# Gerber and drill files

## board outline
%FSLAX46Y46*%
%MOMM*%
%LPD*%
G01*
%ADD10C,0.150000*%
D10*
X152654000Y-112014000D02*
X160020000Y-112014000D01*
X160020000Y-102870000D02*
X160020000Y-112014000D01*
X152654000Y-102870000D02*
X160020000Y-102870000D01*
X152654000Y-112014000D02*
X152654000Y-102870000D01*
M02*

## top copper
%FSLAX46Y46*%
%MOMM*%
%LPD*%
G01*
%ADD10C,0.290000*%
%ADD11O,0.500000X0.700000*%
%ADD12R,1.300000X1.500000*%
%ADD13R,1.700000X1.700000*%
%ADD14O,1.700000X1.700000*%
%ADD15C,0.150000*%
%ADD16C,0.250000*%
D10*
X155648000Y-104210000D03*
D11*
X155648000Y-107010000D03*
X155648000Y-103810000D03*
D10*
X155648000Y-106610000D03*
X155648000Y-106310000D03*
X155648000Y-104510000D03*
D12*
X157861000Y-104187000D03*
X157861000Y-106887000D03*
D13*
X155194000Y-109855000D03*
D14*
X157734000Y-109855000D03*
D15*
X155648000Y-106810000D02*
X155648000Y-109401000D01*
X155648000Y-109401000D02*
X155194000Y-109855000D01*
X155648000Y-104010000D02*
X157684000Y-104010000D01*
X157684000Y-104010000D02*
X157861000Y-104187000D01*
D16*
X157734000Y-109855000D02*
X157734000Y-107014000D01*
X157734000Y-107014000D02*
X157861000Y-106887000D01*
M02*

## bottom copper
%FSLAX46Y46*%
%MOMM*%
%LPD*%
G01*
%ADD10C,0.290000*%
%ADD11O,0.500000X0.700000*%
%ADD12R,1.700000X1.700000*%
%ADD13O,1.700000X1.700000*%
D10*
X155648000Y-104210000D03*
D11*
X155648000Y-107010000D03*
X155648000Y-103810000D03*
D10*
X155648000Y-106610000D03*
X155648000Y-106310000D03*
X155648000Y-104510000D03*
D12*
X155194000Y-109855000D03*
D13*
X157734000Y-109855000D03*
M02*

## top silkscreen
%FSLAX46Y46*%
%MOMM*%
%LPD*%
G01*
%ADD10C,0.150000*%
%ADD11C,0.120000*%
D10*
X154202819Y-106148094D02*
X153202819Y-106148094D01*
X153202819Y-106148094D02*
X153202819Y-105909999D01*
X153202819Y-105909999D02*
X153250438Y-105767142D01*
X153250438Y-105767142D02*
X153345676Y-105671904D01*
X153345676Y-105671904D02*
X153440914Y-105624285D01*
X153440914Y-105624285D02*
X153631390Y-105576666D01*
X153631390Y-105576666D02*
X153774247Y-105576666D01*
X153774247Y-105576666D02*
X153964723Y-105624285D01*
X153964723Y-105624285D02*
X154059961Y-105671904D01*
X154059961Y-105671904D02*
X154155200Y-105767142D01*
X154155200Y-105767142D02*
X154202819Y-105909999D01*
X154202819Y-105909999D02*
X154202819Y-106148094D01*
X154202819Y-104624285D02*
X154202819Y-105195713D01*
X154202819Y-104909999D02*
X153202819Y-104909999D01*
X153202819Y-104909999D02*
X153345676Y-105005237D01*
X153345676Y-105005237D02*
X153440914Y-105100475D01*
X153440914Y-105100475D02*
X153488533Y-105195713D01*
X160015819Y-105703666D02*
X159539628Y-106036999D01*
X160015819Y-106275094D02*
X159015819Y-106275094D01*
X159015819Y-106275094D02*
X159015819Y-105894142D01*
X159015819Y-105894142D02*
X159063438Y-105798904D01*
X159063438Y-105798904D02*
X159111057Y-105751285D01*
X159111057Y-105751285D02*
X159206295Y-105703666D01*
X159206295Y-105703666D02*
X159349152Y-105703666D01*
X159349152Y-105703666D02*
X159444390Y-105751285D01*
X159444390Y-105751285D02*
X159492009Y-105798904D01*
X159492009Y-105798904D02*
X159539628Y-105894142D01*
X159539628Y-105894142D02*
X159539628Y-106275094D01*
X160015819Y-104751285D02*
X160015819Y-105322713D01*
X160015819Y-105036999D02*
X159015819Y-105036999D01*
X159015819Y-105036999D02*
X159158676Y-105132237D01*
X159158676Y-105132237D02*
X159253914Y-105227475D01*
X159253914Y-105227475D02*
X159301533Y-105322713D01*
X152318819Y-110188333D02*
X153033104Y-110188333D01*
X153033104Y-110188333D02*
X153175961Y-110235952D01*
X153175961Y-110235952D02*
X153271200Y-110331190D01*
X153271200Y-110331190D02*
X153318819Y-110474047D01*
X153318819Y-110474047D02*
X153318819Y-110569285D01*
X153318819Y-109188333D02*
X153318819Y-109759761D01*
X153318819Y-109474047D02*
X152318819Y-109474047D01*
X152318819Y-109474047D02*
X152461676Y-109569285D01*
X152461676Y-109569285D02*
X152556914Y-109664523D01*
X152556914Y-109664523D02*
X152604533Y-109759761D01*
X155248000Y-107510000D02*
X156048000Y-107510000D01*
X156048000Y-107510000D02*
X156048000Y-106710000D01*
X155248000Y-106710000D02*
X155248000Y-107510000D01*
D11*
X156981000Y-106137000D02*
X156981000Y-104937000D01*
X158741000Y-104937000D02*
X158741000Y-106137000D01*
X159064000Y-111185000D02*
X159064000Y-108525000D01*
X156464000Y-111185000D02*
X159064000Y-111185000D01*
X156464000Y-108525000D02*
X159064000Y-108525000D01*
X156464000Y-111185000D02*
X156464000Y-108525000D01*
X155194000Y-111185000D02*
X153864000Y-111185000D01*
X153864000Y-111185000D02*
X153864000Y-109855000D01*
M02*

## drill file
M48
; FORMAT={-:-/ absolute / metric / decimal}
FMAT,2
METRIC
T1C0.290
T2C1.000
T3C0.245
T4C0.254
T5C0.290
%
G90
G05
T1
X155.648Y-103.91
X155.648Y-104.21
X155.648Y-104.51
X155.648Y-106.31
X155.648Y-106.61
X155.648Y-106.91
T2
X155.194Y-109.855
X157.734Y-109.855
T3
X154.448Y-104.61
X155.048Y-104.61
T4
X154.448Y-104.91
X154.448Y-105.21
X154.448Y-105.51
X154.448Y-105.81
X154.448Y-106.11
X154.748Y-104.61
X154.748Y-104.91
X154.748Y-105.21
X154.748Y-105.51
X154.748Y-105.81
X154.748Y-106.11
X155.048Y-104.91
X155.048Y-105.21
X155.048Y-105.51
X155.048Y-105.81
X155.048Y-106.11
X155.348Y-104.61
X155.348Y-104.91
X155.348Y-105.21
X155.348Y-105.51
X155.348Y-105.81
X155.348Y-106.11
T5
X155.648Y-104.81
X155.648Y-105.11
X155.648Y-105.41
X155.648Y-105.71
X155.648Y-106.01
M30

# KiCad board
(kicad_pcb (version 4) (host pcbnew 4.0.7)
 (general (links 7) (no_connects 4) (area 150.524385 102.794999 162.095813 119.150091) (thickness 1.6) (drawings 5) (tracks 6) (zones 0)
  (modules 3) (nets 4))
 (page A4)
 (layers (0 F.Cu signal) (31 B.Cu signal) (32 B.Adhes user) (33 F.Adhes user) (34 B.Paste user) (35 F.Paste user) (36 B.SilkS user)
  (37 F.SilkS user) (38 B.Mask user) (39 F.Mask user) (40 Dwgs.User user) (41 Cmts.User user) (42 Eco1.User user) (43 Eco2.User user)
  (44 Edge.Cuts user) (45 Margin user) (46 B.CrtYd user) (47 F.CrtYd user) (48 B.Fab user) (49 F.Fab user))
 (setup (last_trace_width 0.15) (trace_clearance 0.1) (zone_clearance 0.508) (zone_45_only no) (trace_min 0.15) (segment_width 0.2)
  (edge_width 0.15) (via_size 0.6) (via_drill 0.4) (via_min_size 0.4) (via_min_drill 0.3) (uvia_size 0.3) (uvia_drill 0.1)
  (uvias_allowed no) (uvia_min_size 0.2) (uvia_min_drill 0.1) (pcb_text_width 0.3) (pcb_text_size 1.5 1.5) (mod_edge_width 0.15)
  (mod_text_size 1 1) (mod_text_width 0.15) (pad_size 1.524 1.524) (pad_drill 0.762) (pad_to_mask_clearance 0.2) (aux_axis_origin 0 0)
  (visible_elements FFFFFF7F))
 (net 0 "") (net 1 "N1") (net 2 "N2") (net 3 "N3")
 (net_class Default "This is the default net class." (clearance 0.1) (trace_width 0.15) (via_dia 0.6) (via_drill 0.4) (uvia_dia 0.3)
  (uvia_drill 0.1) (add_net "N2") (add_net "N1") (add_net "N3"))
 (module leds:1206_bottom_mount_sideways (layer F.Cu) (at 155.448 105.41 90)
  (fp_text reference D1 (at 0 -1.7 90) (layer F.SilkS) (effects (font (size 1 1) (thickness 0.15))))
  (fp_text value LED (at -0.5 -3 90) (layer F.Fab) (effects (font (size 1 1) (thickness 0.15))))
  (fp_line (start -2.1 -0.2) (end -2.1 0.6) (layer F.SilkS) (width 0.15))
  (fp_line (start -2.1 0.6) (end -1.3 0.6) (layer F.SilkS) (width 0.15))
  (fp_line (start -1.3 -0.2) (end -2.1 -0.2) (layer F.SilkS) (width 0.15))
  (pad 2 thru_hole circle (at 1.2 0.2 270) (size 0.29 0.29) (drill 0.29) (layers *.Cu *.Mask) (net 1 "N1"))
  (pad "" np_thru_hole circle (at 0.8 -0.7 270) (size 0.254 0.254) (drill 0.254) (layers *.Cu *.Mask))
  (pad "" np_thru_hole circle (at 0.5 -0.7 270) (size 0.254 0.254) (drill 0.254) (layers *.Cu *.Mask))
  (pad "" np_thru_hole circle (at 0.2 -0.7 270) (size 0.254 0.254) (drill 0.254) (layers *.Cu *.Mask))
  (pad "" np_thru_hole circle (at -0.1 -0.7 270) (size 0.254 0.254) (drill 0.254) (layers *.Cu *.Mask))
  (pad "" np_thru_hole circle (at -0.4 -0.7 270) (size 0.254 0.254) (drill 0.254) (layers *.Cu *.Mask))
  (pad "" np_thru_hole circle (at -0.7 -0.7 270) (size 0.254 0.254) (drill 0.254) (layers *.Cu *.Mask))
  (pad "" np_thru_hole circle (at 0.8 -0.4 270) (size 0.245 0.245) (drill 0.245) (layers *.Cu *.Mask))
  (pad 1 thru_hole oval (at -1.5 0.2 270) (size 0.7 0.5) (drill 0.29 (offset 0.1 0)) (layers *.Cu *.Mask) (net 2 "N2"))
  (pad 2 thru_hole oval (at 1.5 0.2 90) (size 0.7 0.5) (drill oval 0.29 (offset 0.1 0)) (layers *.Cu *.Mask) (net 1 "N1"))
  (pad "" np_thru_hole circle (at 0.8 -1 270) (size 0.245 0.245) (drill 0.245) (layers *.Cu *.Mask))
  (pad "" np_thru_hole circle (at 0.8 -0.1 270) (size 0.254 0.254) (drill 0.254) (layers *.Cu *.Mask))
  (pad "" np_thru_hole circle (at 0.5 -1 270) (size 0.254 0.254) (drill 0.254) (layers *.Cu *.Mask))
  (pad "" np_thru_hole circle (at 0.5 -0.4 270) (size 0.254 0.254) (drill 0.254) (layers *.Cu *.Mask))
  (pad "" np_thru_hole circle (at 0.5 -0.1 270) (size 0.254 0.254) (drill 0.254) (layers *.Cu *.Mask))
  (pad "" np_thru_hole circle (at 0.2 -1 270) (size 0.254 0.254) (drill 0.254) (layers *.Cu *.Mask))
  (pad "" np_thru_hole circle (at 0.2 -0.4 270) (size 0.254 0.254) (drill 0.254) (layers *.Cu *.Mask))
  (pad "" np_thru_hole circle (at 0.2 -0.1 270) (size 0.254 0.254) (drill 0.254) (layers *.Cu *.Mask))
  (pad "" np_thru_hole circle (at -0.1 -1 270) (size 0.254 0.254) (drill 0.254) (layers *.Cu *.Mask))
  (pad "" np_thru_hole circle (at -0.1 -0.4 270) (size 0.254 0.254) (drill 0.254) (layers *.Cu *.Mask))
  (pad "" np_thru_hole circle (at -0.1 -0.1 270) (size 0.254 0.254) (drill 0.254) (layers *.Cu *.Mask))
  (pad "" np_thru_hole circle (at -0.4 -1 270) (size 0.254 0.254) (drill 0.254) (layers *.Cu *.Mask))
  (pad "" np_thru_hole circle (at -0.4 -0.4 270) (size 0.254 0.254) (drill 0.254) (layers *.Cu *.Mask))
  (pad "" np_thru_hole circle (at -0.4 -0.1 270) (size 0.254 0.254) (drill 0.254) (layers *.Cu *.Mask))
  (pad "" np_thru_hole circle (at -0.7 -1 270) (size 0.254 0.254) (drill 0.254) (layers *.Cu *.Mask))
  (pad "" np_thru_hole circle (at -0.7 -0.4 270) (size 0.254 0.254) (drill 0.254) (layers *.Cu *.Mask))
  (pad "" np_thru_hole circle (at -0.7 -0.1 270) (size 0.254 0.254) (drill 0.254) (layers *.Cu *.Mask))
  (pad 1 thru_hole circle (at -1.2 0.2 270) (size 0.29 0.29) (drill 0.29) (layers *.Cu *.Mask) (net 2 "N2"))
  (pad 1 thru_hole circle (at -0.9 0.2 270) (size 0.29 0.29) (drill 0.29) (layers *.Cu *.Mask) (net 2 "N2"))
  (pad "" np_thru_hole circle (at -0.6 0.2 270) (size 0.29 0.29) (drill 0.29) (layers *.Cu *.Mask))
  (pad "" np_thru_hole circle (at -0.3 0.2 270) (size 0.29 0.29) (drill 0.29) (layers *.Cu *.Mask))
  (pad "" np_thru_hole circle (at 0 0.2 270) (size 0.29 0.29) (drill 0.29) (layers *.Cu *.Mask))
  (pad "" np_thru_hole circle (at 0.3 0.2 270) (size 0.29 0.29) (drill 0.29) (layers *.Cu *.Mask))
  (pad "" np_thru_hole circle (at 0.6 0.2 270) (size 0.29 0.29) (drill 0.29) (layers *.Cu *.Mask))
  (pad 2 thru_hole circle (at 0.9 0.2 270) (size 0.29 0.29) (drill 0.29) (layers *.Cu *.Mask) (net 1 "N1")))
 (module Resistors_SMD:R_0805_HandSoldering (layer F.Cu) (at 157.861 105.537 270)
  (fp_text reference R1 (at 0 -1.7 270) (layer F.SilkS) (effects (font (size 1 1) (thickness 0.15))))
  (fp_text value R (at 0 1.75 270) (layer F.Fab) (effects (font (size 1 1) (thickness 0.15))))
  (fp_line (start 0.6 0.88) (end -0.6 0.88) (layer F.SilkS) (width 0.12))
  (fp_line (start -0.6 -0.88) (end 0.6 -0.88) (layer F.SilkS) (width 0.12))
  (pad 1 smd rect (at -1.35 0 270) (size 1.5 1.3) (layers F.Cu F.Paste F.Mask) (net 1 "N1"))
  (pad 2 smd rect (at 1.35 0 270) (size 1.5 1.3) (layers F.Cu F.Paste F.Mask) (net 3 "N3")))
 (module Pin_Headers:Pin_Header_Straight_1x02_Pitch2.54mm (layer F.Cu) (at 155.194 109.855 90)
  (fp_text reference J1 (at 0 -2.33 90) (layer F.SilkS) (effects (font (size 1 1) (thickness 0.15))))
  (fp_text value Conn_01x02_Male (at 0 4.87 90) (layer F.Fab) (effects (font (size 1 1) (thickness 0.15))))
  (fp_line (start -1.33 3.87) (end 1.33 3.87) (layer F.SilkS) (width 0.12))
  (fp_line (start -1.33 1.27) (end -1.33 3.87) (layer F.SilkS) (width 0.12))
  (fp_line (start 1.33 1.27) (end 1.33 3.87) (layer F.SilkS) (width 0.12))
  (fp_line (start -1.33 1.27) (end 1.33 1.27) (layer F.SilkS) (width 0.12))
  (fp_line (start -1.33 0) (end -1.33 -1.33) (layer F.SilkS) (width 0.12))
  (fp_line (start -1.33 -1.33) (end 0 -1.33) (layer F.SilkS) (width 0.12))
  (pad 1 thru_hole rect (at 0 0 90) (size 1.7 1.7) (drill 1) (layers *.Cu *.Mask) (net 2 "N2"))
  (pad 2 thru_hole oval (at 0 2.54 90) (size 1.7 1.7) (drill 1) (layers *.Cu *.Mask) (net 3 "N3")))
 (gr_line (start 152.654 112.014) (end 160.02 112.014) (angle 90) (layer Edge.Cuts) (width 0.15))
 (gr_line (start 160.02 102.87) (end 160.02 112.014) (angle 90) (layer Edge.Cuts) (width 0.15))
 (gr_line (start 152.654 102.87) (end 160.02 102.87) (angle 90) (layer Edge.Cuts) (width 0.15))
 (gr_line (start 152.654 112.014) (end 152.654 102.87) (angle 90) (layer Edge.Cuts) (width 0.15))
 (segment (start 155.648 106.81) (end 155.648 109.401) (width 0.15) (layer F.Cu) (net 2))
 (segment (start 155.648 109.401) (end 155.194 109.855) (width 0.15) (layer F.Cu) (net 2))
 (segment (start 155.648 104.01) (end 157.684 104.01) (width 0.15) (layer F.Cu) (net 1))
 (segment (start 157.684 104.01) (end 157.861 104.187) (width 0.15) (layer F.Cu) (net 1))
 (segment (start 157.734 109.855) (end 157.734 107.014) (width 0.25) (layer F.Cu) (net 3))
 (segment (start 157.734 107.014) (end 157.861 106.887) (width 0.25) (layer F.Cu) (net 3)))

